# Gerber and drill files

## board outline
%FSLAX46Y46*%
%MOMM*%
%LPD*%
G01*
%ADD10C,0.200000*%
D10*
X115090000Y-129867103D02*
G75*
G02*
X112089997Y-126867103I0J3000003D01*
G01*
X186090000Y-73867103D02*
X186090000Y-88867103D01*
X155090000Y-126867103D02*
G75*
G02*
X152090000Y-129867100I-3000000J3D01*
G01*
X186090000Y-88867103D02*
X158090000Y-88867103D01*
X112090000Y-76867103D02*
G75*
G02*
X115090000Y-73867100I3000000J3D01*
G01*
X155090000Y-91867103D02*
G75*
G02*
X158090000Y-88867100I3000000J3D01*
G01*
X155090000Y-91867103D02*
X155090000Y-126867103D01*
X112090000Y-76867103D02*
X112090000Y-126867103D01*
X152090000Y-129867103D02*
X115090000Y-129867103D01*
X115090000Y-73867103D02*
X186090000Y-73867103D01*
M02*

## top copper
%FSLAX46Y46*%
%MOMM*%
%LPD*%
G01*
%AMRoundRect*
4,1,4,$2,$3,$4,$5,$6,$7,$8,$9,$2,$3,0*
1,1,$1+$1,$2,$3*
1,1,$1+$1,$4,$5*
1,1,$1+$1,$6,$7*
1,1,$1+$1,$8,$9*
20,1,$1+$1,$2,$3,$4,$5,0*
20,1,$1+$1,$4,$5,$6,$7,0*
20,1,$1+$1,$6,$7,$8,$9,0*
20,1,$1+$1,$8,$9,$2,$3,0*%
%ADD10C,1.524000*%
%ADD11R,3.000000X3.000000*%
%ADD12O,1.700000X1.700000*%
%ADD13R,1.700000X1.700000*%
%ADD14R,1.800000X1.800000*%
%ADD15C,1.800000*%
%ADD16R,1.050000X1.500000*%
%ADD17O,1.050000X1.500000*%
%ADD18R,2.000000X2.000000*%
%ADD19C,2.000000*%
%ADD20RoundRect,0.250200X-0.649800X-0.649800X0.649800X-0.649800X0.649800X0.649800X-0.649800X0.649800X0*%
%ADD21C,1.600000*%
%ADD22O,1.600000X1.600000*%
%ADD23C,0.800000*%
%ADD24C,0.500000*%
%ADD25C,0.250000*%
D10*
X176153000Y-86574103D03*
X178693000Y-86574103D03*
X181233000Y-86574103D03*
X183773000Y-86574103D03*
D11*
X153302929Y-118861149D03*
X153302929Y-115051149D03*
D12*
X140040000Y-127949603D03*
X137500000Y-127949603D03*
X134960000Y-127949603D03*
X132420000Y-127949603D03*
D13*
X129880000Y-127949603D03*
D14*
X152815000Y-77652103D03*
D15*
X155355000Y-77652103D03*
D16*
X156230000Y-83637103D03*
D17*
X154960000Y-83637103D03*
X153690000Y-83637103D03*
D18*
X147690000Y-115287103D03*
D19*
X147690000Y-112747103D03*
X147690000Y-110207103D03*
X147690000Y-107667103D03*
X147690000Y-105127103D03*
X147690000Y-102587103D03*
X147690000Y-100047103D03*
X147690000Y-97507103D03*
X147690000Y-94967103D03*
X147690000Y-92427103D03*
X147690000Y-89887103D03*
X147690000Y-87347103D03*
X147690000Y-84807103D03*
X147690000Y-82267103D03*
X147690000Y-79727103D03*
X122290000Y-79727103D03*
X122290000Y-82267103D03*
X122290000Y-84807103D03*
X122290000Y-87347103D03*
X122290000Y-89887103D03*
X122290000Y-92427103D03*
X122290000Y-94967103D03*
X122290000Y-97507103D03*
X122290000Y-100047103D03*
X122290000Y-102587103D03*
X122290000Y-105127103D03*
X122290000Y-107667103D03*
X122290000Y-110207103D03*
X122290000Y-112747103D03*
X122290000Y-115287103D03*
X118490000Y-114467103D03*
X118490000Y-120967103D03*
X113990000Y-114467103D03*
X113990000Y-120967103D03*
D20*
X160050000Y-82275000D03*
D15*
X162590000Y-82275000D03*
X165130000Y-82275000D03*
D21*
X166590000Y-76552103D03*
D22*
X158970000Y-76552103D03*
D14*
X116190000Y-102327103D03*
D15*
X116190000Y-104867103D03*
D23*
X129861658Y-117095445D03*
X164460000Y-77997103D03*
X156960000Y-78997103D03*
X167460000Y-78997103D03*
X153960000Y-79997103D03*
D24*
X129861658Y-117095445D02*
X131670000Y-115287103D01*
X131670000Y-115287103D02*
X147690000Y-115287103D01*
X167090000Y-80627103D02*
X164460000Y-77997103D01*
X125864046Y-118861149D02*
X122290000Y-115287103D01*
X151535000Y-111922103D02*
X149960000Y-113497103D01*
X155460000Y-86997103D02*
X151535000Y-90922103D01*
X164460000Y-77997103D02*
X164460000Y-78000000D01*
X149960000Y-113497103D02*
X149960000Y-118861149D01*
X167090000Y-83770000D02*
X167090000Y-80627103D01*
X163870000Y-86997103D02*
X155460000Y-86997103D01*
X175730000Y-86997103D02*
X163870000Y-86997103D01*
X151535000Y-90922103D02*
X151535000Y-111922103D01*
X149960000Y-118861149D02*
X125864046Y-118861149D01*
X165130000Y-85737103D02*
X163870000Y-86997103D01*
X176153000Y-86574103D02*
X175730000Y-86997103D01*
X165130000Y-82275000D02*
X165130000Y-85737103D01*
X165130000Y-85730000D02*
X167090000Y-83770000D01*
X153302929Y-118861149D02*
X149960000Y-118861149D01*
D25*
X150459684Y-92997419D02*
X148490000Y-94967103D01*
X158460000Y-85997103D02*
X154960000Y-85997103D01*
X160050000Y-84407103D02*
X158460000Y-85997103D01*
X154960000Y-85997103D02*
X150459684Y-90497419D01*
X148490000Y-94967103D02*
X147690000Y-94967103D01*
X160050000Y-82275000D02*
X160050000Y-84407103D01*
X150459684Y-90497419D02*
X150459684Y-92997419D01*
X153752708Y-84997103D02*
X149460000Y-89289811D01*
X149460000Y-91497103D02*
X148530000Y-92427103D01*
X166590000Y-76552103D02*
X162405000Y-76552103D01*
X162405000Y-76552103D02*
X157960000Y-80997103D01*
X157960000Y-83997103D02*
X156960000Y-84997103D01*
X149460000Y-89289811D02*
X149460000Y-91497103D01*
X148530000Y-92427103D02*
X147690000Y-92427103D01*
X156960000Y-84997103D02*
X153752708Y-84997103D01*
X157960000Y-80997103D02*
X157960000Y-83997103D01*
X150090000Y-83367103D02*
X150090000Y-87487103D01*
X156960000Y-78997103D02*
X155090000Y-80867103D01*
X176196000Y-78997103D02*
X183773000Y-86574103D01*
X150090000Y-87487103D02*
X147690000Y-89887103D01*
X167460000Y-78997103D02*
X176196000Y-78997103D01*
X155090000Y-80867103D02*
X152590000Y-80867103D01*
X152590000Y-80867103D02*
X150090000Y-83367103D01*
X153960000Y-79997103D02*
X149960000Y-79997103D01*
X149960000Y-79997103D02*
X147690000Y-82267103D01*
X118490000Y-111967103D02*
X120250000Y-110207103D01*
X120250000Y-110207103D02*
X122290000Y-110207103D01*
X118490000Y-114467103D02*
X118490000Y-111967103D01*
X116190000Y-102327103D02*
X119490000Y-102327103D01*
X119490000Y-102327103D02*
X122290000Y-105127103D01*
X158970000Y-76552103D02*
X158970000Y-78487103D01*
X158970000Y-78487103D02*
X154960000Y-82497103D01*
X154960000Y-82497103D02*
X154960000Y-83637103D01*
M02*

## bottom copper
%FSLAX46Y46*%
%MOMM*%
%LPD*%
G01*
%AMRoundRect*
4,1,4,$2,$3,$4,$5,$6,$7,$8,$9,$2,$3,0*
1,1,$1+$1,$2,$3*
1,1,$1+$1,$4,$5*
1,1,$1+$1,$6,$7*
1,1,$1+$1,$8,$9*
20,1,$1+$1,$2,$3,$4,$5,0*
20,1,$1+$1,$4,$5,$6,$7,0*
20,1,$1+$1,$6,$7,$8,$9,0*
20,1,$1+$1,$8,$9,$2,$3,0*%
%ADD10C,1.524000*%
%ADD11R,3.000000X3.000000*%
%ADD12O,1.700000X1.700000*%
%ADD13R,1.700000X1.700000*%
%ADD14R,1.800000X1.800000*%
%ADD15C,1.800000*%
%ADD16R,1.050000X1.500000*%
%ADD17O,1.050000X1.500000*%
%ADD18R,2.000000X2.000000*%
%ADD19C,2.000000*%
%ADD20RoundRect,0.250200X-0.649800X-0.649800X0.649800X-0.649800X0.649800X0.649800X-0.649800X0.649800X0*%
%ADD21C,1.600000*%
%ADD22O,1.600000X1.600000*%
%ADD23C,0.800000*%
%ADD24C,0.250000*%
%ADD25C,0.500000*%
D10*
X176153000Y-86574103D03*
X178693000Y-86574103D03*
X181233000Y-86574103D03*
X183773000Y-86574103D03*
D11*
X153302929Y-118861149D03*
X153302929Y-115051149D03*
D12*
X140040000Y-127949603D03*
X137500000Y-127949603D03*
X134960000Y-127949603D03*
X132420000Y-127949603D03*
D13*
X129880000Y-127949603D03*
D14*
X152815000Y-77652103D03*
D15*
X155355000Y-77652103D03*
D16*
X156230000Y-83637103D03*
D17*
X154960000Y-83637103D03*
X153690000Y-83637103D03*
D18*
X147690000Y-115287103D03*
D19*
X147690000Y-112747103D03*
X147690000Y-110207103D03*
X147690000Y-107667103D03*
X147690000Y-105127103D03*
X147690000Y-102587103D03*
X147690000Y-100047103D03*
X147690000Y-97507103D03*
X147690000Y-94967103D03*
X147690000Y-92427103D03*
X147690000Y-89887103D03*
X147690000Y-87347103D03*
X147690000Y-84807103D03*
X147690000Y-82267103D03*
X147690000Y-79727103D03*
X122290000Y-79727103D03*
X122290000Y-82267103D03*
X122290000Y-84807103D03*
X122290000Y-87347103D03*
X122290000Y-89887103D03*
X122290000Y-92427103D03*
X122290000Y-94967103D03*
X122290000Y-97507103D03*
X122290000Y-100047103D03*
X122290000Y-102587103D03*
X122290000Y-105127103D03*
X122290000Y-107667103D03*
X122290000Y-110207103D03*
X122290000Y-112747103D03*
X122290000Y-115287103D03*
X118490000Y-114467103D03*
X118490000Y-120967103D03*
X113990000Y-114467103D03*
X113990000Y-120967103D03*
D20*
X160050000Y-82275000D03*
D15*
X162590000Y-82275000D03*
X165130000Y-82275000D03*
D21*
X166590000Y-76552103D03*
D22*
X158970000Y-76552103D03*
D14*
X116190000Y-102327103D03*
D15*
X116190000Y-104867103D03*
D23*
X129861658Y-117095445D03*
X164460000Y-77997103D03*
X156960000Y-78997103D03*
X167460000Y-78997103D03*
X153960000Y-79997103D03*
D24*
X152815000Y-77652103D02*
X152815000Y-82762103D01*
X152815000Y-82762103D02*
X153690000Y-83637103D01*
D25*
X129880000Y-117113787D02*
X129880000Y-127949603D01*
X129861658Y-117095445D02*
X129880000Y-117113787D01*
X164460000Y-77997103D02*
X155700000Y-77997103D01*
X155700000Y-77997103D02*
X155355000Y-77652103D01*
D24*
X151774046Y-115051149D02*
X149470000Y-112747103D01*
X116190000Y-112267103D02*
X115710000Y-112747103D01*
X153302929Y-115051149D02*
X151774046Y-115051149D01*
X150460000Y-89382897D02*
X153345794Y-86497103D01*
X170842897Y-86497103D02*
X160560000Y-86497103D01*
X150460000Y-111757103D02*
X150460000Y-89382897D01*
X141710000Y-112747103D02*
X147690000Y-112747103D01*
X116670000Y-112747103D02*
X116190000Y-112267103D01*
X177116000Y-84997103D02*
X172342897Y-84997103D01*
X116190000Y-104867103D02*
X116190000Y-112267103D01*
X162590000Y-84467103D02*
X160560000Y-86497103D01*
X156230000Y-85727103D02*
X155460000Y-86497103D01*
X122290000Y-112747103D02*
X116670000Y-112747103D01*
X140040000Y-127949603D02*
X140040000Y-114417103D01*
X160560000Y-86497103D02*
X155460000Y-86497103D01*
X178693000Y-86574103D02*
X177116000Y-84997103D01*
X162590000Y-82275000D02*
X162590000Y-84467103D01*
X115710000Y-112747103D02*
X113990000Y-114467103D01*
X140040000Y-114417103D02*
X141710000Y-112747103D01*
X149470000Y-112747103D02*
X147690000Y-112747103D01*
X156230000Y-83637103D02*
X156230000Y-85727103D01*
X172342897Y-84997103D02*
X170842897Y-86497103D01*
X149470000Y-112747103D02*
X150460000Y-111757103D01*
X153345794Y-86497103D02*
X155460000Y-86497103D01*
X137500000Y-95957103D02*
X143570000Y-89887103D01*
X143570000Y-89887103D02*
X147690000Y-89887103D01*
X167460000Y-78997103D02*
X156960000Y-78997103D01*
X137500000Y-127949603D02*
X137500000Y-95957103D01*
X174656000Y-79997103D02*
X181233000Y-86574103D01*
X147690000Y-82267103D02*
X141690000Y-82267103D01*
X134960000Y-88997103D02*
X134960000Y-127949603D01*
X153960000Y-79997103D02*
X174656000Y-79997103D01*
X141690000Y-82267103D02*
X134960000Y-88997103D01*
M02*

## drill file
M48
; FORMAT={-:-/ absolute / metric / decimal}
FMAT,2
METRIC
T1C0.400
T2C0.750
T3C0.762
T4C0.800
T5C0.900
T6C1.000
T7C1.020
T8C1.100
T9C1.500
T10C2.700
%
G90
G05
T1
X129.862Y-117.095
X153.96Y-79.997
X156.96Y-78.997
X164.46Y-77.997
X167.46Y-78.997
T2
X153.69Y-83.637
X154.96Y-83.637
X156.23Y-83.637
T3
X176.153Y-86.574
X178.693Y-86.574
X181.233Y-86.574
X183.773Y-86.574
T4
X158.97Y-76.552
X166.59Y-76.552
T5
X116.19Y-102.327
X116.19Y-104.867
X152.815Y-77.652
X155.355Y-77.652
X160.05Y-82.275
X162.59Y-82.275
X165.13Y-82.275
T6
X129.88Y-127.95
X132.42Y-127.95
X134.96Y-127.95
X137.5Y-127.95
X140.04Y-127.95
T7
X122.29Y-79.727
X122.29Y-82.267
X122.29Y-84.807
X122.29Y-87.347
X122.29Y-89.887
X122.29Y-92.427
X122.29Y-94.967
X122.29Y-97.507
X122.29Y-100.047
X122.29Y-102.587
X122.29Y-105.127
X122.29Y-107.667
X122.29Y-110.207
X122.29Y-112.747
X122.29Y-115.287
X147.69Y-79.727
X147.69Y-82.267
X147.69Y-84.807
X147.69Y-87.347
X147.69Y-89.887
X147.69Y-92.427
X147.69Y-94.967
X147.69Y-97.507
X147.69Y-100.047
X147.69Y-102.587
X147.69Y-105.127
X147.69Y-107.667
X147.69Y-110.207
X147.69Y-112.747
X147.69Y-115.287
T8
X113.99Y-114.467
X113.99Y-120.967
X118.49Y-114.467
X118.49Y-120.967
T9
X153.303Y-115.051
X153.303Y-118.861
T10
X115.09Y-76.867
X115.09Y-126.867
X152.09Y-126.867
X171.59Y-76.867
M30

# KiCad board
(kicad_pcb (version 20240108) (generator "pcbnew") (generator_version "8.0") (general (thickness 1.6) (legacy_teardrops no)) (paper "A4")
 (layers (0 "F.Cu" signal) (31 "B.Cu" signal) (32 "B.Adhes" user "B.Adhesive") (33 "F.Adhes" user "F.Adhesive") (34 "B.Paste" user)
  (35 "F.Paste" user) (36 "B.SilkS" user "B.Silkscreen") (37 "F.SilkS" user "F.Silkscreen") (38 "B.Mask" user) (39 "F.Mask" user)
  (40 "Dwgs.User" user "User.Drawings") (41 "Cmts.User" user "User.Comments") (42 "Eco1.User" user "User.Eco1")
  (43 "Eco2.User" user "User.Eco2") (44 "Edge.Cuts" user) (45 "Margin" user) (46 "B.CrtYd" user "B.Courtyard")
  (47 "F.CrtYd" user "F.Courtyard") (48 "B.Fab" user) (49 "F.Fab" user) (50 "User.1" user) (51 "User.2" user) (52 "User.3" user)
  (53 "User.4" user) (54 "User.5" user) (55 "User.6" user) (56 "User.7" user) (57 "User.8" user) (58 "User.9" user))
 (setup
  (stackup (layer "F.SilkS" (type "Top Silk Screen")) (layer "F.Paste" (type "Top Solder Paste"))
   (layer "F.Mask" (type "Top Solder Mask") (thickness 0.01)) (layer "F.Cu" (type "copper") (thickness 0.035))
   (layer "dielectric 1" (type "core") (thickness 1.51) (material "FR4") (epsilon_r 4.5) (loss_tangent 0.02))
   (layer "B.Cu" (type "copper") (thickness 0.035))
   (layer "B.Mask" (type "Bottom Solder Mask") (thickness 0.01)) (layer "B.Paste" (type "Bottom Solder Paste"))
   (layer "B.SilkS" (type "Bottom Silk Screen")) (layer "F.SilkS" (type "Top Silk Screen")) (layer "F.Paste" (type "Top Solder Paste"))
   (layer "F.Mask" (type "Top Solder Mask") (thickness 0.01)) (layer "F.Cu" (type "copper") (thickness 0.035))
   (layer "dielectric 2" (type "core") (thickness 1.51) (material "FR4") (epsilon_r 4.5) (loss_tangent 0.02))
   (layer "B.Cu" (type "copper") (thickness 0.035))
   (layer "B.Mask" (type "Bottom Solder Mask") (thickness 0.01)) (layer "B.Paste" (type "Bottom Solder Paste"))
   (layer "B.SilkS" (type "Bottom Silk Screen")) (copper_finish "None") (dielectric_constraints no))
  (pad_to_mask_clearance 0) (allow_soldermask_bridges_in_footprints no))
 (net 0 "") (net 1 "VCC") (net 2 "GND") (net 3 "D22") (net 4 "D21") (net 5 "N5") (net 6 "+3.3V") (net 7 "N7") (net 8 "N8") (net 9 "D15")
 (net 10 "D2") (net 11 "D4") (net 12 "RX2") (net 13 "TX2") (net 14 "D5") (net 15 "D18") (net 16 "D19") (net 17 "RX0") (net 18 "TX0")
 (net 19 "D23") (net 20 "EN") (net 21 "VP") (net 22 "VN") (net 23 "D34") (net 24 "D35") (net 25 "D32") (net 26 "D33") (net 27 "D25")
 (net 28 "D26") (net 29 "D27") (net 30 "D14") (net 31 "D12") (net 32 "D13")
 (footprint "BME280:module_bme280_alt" (layer "F.Cu") (at 183.773 86.574103 90)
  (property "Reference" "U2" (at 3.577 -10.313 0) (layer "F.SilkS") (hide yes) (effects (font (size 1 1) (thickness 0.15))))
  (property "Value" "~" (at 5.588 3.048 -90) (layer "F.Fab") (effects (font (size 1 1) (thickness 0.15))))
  (pad "1" thru_hole circle (at 0 -7.62 90) (size 1.524 1.524) (drill 0.762) (layers "*.Cu" "*.Mask") (remove_unused_layers no)
   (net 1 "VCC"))
  (pad "2" thru_hole circle (at 0 -5.08 90) (size 1.524 1.524) (drill 0.762) (layers "*.Cu" "*.Mask") (remove_unused_layers no)
   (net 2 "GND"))
  (pad "3" thru_hole circle (at 0 -2.54 90) (size 1.524 1.524) (drill 0.762) (layers "*.Cu" "*.Mask") (remove_unused_layers no)
   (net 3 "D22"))
  (pad "4" thru_hole circle (at 0 0 90) (size 1.524 1.524) (drill 0.762) (layers "*.Cu" "*.Mask") (remove_unused_layers no) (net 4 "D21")))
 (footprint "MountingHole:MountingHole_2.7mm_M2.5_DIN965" (layer "F.Cu") (at 115.09 76.867103)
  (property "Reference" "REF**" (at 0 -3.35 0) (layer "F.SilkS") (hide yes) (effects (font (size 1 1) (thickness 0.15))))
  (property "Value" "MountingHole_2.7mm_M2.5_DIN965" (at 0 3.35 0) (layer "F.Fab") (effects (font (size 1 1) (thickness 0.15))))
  (pad "" np_thru_hole circle (at 0 0) (size 2.7 2.7) (drill 2.7) (layers "F&B.Cu" "*.Mask")))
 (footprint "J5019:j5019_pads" (layer "F.Cu") (at 149.492929 116.321149 90)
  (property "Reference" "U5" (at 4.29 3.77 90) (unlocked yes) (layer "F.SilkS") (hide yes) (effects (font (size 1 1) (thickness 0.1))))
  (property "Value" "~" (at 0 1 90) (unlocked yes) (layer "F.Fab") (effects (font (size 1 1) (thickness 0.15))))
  (pad "3" thru_hole rect (at -2.54 3.81 180) (size 3 3) (drill 1.5) (layers "*.Cu" "*.Mask") (remove_unused_layers no) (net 1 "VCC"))
  (pad "4" thru_hole rect (at 1.27 3.81 180) (size 3 3) (drill 1.5) (layers "*.Cu" "*.Mask") (remove_unused_layers no) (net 2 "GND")))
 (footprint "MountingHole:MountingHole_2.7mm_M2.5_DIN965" (layer "F.Cu") (at 171.59 76.867103)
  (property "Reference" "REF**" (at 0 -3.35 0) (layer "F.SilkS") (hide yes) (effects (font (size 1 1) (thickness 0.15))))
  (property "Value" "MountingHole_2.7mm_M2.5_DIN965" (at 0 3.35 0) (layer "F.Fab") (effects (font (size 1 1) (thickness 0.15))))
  (pad "" np_thru_hole circle (at 0 0) (size 2.7 2.7) (drill 2.7) (layers "F&B.Cu" "*.Mask")))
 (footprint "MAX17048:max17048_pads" (layer "F.Cu") (at 136.23 131.759603 180)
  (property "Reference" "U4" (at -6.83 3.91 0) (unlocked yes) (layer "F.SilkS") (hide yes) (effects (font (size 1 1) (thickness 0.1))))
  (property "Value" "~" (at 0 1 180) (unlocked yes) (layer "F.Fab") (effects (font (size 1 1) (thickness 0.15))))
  (pad "1" thru_hole oval (at -3.81 3.81 270) (size 1.7 1.7) (drill 1) (layers "*.Cu" "*.Mask") (remove_unused_layers no) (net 2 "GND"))
  (pad "2" thru_hole oval (at -1.27 3.81 270) (size 1.7 1.7) (drill 1) (layers "*.Cu" "*.Mask") (remove_unused_layers no) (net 4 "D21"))
  (pad "3" thru_hole oval (at 1.27 3.81 270) (size 1.7 1.7) (drill 1) (layers "*.Cu" "*.Mask") (remove_unused_layers no) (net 3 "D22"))
  (pad "4" thru_hole oval (at 3.81 3.81 270) (size 1.7 1.7) (drill 1) (layers "*.Cu" "*.Mask") (remove_unused_layers no) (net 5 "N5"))
  (pad "5" thru_hole rect (at 6.35 3.81 270) (size 1.7 1.7) (drill 1) (layers "*.Cu" "*.Mask") (remove_unused_layers no) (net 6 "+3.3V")))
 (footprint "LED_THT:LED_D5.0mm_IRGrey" (layer "F.Cu") (at 152.815 77.652103)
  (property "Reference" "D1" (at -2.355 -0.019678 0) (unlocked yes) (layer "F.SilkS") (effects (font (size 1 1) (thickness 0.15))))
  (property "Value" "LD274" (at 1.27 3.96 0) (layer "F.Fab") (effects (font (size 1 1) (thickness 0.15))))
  (pad "1" thru_hole rect (at 0 0) (size 1.8 1.8) (drill 0.9) (layers "*.Cu" "*.Mask") (remove_unused_layers no) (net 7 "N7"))
  (pad "2" thru_hole circle (at 2.54 0) (size 1.8 1.8) (drill 0.9) (layers "*.Cu" "*.Mask") (remove_unused_layers no) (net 1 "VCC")))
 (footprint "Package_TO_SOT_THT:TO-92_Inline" (layer "F.Cu") (at 156.23 83.637103 180)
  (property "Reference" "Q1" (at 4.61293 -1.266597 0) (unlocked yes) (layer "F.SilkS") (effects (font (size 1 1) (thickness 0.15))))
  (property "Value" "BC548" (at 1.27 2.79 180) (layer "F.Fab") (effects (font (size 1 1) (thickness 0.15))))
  (pad "1" thru_hole rect (at 0 0 180) (size 1.05 1.5) (drill 0.75) (layers "*.Cu" "*.Mask") (remove_unused_layers no) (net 2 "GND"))
  (pad "2" thru_hole oval (at 1.27 0 180) (size 1.05 1.5) (drill 0.75) (layers "*.Cu" "*.Mask") (remove_unused_layers no) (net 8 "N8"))
  (pad "3" thru_hole oval (at 2.54 0 180) (size 1.05 1.5) (drill 0.75) (layers "*.Cu" "*.Mask") (remove_unused_layers no) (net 7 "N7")))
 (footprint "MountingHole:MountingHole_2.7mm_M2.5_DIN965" (layer "F.Cu") (at 115.09 126.867103)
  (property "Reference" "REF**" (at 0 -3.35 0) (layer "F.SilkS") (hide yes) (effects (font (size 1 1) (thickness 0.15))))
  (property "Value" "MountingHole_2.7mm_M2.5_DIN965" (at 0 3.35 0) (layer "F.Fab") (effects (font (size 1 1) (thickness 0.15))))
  (pad "" np_thru_hole circle (at 0 0) (size 2.7 2.7) (drill 2.7) (layers "F&B.Cu" "*.Mask")))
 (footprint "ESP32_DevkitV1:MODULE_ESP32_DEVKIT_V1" (layer "F.Cu") (at 134.99 99.772103 180)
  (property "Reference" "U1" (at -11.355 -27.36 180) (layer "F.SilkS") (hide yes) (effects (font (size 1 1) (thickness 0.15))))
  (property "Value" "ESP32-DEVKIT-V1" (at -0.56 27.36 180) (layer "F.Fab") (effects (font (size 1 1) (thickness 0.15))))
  (pad "1" thru_hole rect (at -12.7 -15.515 180) (size 2 2) (drill 1.02) (layers "*.Cu" "*.Mask") (remove_unused_layers no) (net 6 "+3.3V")
   (solder_mask_margin 0.102))
  (pad "2" thru_hole circle (at -12.7 -12.975 180) (size 2 2) (drill 1.02) (layers "*.Cu" "*.Mask") (remove_unused_layers no) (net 2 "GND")
   (solder_mask_margin 0.102))
  (pad "3" thru_hole circle (at -12.7 -10.435 180) (size 2 2) (drill 1.02) (layers "*.Cu" "*.Mask") (remove_unused_layers no) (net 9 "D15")
   (solder_mask_margin 0.102))
  (pad "4" thru_hole circle (at -12.7 -7.895 180) (size 2 2) (drill 1.02) (layers "*.Cu" "*.Mask") (remove_unused_layers no) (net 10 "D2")
   (solder_mask_margin 0.102))
  (pad "5" thru_hole circle (at -12.7 -5.355 180) (size 2 2) (drill 1.02) (layers "*.Cu" "*.Mask") (remove_unused_layers no) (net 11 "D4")
   (solder_mask_margin 0.102))
  (pad "6" thru_hole circle (at -12.7 -2.815 180) (size 2 2) (drill 1.02) (layers "*.Cu" "*.Mask") (remove_unused_layers no) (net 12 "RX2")
   (solder_mask_margin 0.102))
  (pad "7" thru_hole circle (at -12.7 -0.275 180) (size 2 2) (drill 1.02) (layers "*.Cu" "*.Mask") (remove_unused_layers no) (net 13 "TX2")
   (solder_mask_margin 0.102))
  (pad "8" thru_hole circle (at -12.7 2.265 180) (size 2 2) (drill 1.02) (layers "*.Cu" "*.Mask") (remove_unused_layers no) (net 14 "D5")
   (solder_mask_margin 0.102))
  (pad "9" thru_hole circle (at -12.7 4.805 180) (size 2 2) (drill 1.02) (layers "*.Cu" "*.Mask") (remove_unused_layers no) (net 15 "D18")
   (solder_mask_margin 0.102))
  (pad "10" thru_hole circle (at -12.7 7.345 180) (size 2 2) (drill 1.02) (layers "*.Cu" "*.Mask") (remove_unused_layers no) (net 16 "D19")
   (solder_mask_margin 0.102))
  (pad "11" thru_hole circle (at -12.7 9.885 180) (size 2 2) (drill 1.02) (layers "*.Cu" "*.Mask") (remove_unused_layers no) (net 4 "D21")
   (solder_mask_margin 0.102))
  (pad "12" thru_hole circle (at -12.7 12.425 180) (size 2 2) (drill 1.02) (layers "*.Cu" "*.Mask") (remove_unused_layers no) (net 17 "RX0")
   (solder_mask_margin 0.102))
  (pad "13" thru_hole circle (at -12.7 14.965 180) (size 2 2) (drill 1.02) (layers "*.Cu" "*.Mask") (remove_unused_layers no) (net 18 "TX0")
   (solder_mask_margin 0.102))
  (pad "14" thru_hole circle (at -12.7 17.505 180) (size 2 2) (drill 1.02) (layers "*.Cu" "*.Mask") (remove_unused_layers no) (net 3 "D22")
   (solder_mask_margin 0.102))
  (pad "15" thru_hole circle (at -12.7 20.045 180) (size 2 2) (drill 1.02) (layers "*.Cu" "*.Mask") (remove_unused_layers no) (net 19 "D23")
   (solder_mask_margin 0.102))
  (pad "16" thru_hole circle (at 12.7 20.045 180) (size 2 2) (drill 1.02) (layers "*.Cu" "*.Mask") (remove_unused_layers no) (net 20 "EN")
   (solder_mask_margin 0.102))
  (pad "17" thru_hole circle (at 12.7 17.505 180) (size 2 2) (drill 1.02) (layers "*.Cu" "*.Mask") (remove_unused_layers no) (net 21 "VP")
   (solder_mask_margin 0.102))
  (pad "18" thru_hole circle (at 12.7 14.965 180) (size 2 2) (drill 1.02) (layers "*.Cu" "*.Mask") (remove_unused_layers no) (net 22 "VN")
   (solder_mask_margin 0.102))
  (pad "19" thru_hole circle (at 12.7 12.425 180) (size 2 2) (drill 1.02) (layers "*.Cu" "*.Mask") (remove_unused_layers no) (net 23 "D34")
   (solder_mask_margin 0.102))
  (pad "20" thru_hole circle (at 12.7 9.885 180) (size 2 2) (drill 1.02) (layers "*.Cu" "*.Mask") (remove_unused_layers no) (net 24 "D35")
   (solder_mask_margin 0.102))
  (pad "21" thru_hole circle (at 12.7 7.345 180) (size 2 2) (drill 1.02) (layers "*.Cu" "*.Mask") (remove_unused_layers no) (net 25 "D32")
   (solder_mask_margin 0.102))
  (pad "22" thru_hole circle (at 12.7 4.805 180) (size 2 2) (drill 1.02) (layers "*.Cu" "*.Mask") (remove_unused_layers no) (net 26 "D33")
   (solder_mask_margin 0.102))
  (pad "23" thru_hole circle (at 12.7 2.265 180) (size 2 2) (drill 1.02) (layers "*.Cu" "*.Mask") (remove_unused_layers no) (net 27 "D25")
   (solder_mask_margin 0.102))
  (pad "24" thru_hole circle (at 12.7 -0.275 180) (size 2 2) (drill 1.02) (layers "*.Cu" "*.Mask") (remove_unused_layers no) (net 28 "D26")
   (solder_mask_margin 0.102))
  (pad "25" thru_hole circle (at 12.7 -2.815 180) (size 2 2) (drill 1.02) (layers "*.Cu" "*.Mask") (remove_unused_layers no) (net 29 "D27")
   (solder_mask_margin 0.102))
  (pad "26" thru_hole circle (at 12.7 -5.355 180) (size 2 2) (drill 1.02) (layers "*.Cu" "*.Mask") (remove_unused_layers no) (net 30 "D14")
   (solder_mask_margin 0.102))
  (pad "27" thru_hole circle (at 12.7 -7.895 180) (size 2 2) (drill 1.02) (layers "*.Cu" "*.Mask") (remove_unused_layers no) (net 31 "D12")
   (solder_mask_margin 0.102))
  (pad "28" thru_hole circle (at 12.7 -10.435 180) (size 2 2) (drill 1.02) (layers "*.Cu" "*.Mask") (remove_unused_layers no) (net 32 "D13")
   (solder_mask_margin 0.102))
  (pad "29" thru_hole circle (at 12.7 -12.975 180) (size 2 2) (drill 1.02) (layers "*.Cu" "*.Mask") (remove_unused_layers no) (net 2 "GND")
   (solder_mask_margin 0.102))
  (pad "30" thru_hole circle (at 12.7 -15.515 180) (size 2 2) (drill 1.02) (layers "*.Cu" "*.Mask") (remove_unused_layers no) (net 1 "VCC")
   (solder_mask_margin 0.102))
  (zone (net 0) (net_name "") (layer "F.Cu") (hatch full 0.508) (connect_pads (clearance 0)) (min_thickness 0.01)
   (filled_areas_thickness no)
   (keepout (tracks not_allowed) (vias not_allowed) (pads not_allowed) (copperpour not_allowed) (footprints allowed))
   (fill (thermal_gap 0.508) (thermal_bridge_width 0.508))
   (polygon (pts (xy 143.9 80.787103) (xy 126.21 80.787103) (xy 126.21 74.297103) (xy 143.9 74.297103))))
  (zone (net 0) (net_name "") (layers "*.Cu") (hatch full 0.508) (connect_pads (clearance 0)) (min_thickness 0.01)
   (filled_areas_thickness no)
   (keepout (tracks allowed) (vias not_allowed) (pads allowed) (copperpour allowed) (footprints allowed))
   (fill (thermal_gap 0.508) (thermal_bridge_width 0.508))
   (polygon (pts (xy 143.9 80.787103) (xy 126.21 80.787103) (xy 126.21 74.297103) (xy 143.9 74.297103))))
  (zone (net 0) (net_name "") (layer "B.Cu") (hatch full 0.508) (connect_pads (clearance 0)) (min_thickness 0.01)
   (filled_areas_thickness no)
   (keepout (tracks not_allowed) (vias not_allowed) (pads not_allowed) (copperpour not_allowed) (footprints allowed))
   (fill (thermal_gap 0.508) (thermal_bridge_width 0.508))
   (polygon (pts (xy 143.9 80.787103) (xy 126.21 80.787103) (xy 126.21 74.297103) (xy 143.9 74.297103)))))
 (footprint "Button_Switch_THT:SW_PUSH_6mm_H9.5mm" (layer "F.Cu") (at 118.49 114.467103 -90)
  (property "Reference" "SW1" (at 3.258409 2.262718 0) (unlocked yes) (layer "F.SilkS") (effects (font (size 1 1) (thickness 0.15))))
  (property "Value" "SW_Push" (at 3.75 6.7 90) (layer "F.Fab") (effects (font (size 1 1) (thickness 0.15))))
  (pad "1" thru_hole circle (at 0 0) (size 2 2) (drill 1.1) (layers "*.Cu" "*.Mask") (remove_unused_layers no) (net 32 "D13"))
  (pad "1" thru_hole circle (at 6.5 0) (size 2 2) (drill 1.1) (layers "*.Cu" "*.Mask") (remove_unused_layers no) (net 32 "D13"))
  (pad "2" thru_hole circle (at 0 4.5) (size 2 2) (drill 1.1) (layers "*.Cu" "*.Mask") (remove_unused_layers no) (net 2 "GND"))
  (pad "2" thru_hole circle (at 6.5 4.5) (size 2 2) (drill 1.1) (layers "*.Cu" "*.Mask") (remove_unused_layers no) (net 2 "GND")))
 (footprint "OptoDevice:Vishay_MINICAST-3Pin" (layer "F.Cu") (at 160.05 82.275)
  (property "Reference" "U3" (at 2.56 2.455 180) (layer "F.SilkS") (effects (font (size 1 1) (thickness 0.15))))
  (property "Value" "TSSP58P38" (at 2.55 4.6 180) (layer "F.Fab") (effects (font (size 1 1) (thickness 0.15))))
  (pad "1" thru_hole roundrect (at 0 0) (size 1.8 1.8) (drill 0.9) (layers "*.Cu" "*.Mask") (remove_unused_layers no)
   (roundrect_rratio 0.139) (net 15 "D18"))
  (pad "2" thru_hole circle (at 2.54 0) (size 1.8 1.8) (drill 0.9) (layers "*.Cu" "*.Mask") (remove_unused_layers no) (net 2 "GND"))
  (pad "3" thru_hole circle (at 5.08 0) (size 1.8 1.8) (drill 0.9) (layers "*.Cu" "*.Mask") (remove_unused_layers no) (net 1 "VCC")))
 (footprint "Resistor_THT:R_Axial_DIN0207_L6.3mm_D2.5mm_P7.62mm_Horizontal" (layer "F.Cu") (at 166.59 76.552103 180)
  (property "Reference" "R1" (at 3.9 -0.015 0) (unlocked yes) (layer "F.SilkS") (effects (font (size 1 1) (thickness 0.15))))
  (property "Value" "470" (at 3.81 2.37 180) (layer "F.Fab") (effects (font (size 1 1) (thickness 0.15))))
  (pad "1" thru_hole circle (at 0 0 180) (size 1.6 1.6) (drill 0.8) (layers "*.Cu" "*.Mask") (remove_unused_layers no) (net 16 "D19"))
  (pad "2" thru_hole oval (at 7.62 0 180) (size 1.6 1.6) (drill 0.8) (layers "*.Cu" "*.Mask") (remove_unused_layers no) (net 8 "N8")))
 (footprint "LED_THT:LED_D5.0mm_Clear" (layer "F.Cu") (at 116.19 102.327103 -90)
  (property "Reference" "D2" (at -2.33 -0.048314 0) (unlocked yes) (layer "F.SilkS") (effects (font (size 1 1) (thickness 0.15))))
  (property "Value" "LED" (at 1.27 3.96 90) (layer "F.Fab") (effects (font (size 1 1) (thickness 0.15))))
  (pad "1" thru_hole rect (at 0 0 270) (size 1.8 1.8) (drill 0.9) (layers "*.Cu" "*.Mask") (remove_unused_layers no) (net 30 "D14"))
  (pad "2" thru_hole circle (at 2.54 0 270) (size 1.8 1.8) (drill 0.9) (layers "*.Cu" "*.Mask") (remove_unused_layers no) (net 2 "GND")))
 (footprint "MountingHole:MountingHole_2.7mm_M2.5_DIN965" (layer "F.Cu") (at 152.09 126.867103)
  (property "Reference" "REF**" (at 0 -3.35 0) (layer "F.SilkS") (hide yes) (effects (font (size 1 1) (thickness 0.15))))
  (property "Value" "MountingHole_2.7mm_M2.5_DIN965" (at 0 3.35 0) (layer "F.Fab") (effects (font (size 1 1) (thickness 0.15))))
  (pad "" np_thru_hole circle (at 0 0) (size 2.7 2.7) (drill 2.7) (layers "*.Cu" "*.Mask")))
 (gr_arc (start 115.09 129.867103) (mid 112.96868 128.988423) (end 112.09 126.867103) (stroke (width 0.2) (type default))
  (layer "Edge.Cuts"))
 (gr_line (start 186.09 73.867103) (end 186.09 88.867103) (stroke (width 0.2) (type default)) (layer "Edge.Cuts"))
 (gr_arc (start 155.09 126.867103) (mid 154.21132 128.988423) (end 152.09 129.867103) (stroke (width 0.2) (type default))
  (layer "Edge.Cuts"))
 (gr_line (start 186.09 88.867103) (end 158.09 88.867103) (stroke (width 0.2) (type default)) (layer "Edge.Cuts"))
 (gr_arc (start 112.09 76.867103) (mid 112.96868 74.745783) (end 115.09 73.867103) (stroke (width 0.2) (type default)) (layer "Edge.Cuts"))
 (gr_arc (start 155.09 91.867103) (mid 155.96868 89.745783) (end 158.09 88.867103) (stroke (width 0.2) (type default)) (layer "Edge.Cuts"))
 (gr_line (start 155.09 91.867103) (end 155.09 126.867103) (stroke (width 0.2) (type default)) (layer "Edge.Cuts"))
 (gr_line (start 112.09 76.867103) (end 112.09 126.867103) (stroke (width 0.2) (type default)) (layer "Edge.Cuts"))
 (gr_line (start 152.09 129.867103) (end 115.09 129.867103) (stroke (width 0.2) (type default)) (layer "Edge.Cuts"))
 (gr_line (start 115.09 73.867103) (end 186.09 73.867103) (stroke (width 0.2) (type default)) (layer "Edge.Cuts"))
 (segment (start 152.815 77.652103) (end 152.815 82.762103) (width 0.25) (layer "B.Cu") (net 7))
 (segment (start 152.815 82.762103) (end 153.69 83.637103) (width 0.25) (layer "B.Cu") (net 7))
 (segment (start 129.861658 117.095445) (end 131.67 115.287103) (width 0.5) (layer "F.Cu") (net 6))
 (segment (start 131.67 115.287103) (end 147.69 115.287103) (width 0.5) (layer "F.Cu") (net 6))
 (via (at 129.861658 117.095445) (size 0.8) (drill 0.4) (layers "F.Cu" "B.Cu") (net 6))
 (segment (start 129.88 117.113787) (end 129.88 127.949603) (width 0.5) (layer "B.Cu") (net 6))
 (segment (start 129.861658 117.095445) (end 129.88 117.113787) (width 0.5) (layer "B.Cu") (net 6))
 (segment (start 167.09 80.627103) (end 164.46 77.997103) (width 0.5) (layer "F.Cu") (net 1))
 (segment (start 125.864046 118.861149) (end 122.29 115.287103) (width 0.5) (layer "F.Cu") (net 1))
 (segment (start 151.535 111.922103) (end 149.96 113.497103) (width 0.5) (layer "F.Cu") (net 1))
 (segment (start 155.46 86.997103) (end 151.535 90.922103) (width 0.5) (layer "F.Cu") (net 1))
 (segment (start 164.46 77.997103) (end 164.46 78) (width 0.5) (layer "F.Cu") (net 1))
 (segment (start 149.96 113.497103) (end 149.96 118.861149) (width 0.5) (layer "F.Cu") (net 1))
 (segment (start 167.09 83.77) (end 167.09 80.627103) (width 0.5) (layer "F.Cu") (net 1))
 (segment (start 163.87 86.997103) (end 155.46 86.997103) (width 0.5) (layer "F.Cu") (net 1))
 (segment (start 175.73 86.997103) (end 163.87 86.997103) (width 0.5) (layer "F.Cu") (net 1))
 (segment (start 151.535 90.922103) (end 151.535 111.922103) (width 0.5) (layer "F.Cu") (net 1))
 (segment (start 149.96 118.861149) (end 125.864046 118.861149) (width 0.5) (layer "F.Cu") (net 1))
 (segment (start 165.13 85.737103) (end 163.87 86.997103) (width 0.5) (layer "F.Cu") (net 1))
 (segment (start 176.153 86.574103) (end 175.73 86.997103) (width 0.5) (layer "F.Cu") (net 1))
 (segment (start 165.13 82.275) (end 165.13 85.737103) (width 0.5) (layer "F.Cu") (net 1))
 (segment (start 165.13 85.73) (end 167.09 83.77) (width 0.5) (layer "F.Cu") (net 1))
 (segment (start 153.302929 118.861149) (end 149.96 118.861149) (width 0.5) (layer "F.Cu") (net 1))
 (via (at 164.46 77.997103) (size 0.8) (drill 0.4) (layers "F.Cu" "B.Cu") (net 1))
 (segment (start 164.46 77.997103) (end 155.7 77.997103) (width 0.5) (layer "B.Cu") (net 1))
 (segment (start 155.7 77.997103) (end 155.355 77.652103) (width 0.5) (layer "B.Cu") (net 1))
 (segment (start 151.774046 115.051149) (end 149.47 112.747103) (width 0.25) (layer "B.Cu") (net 2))
 (segment (start 116.19 112.267103) (end 115.71 112.747103) (width 0.25) (layer "B.Cu") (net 2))
 (segment (start 153.302929 115.051149) (end 151.774046 115.051149) (width 0.25) (layer "B.Cu") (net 2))
 (segment (start 150.46 89.382897) (end 153.345794 86.497103) (width 0.25) (layer "B.Cu") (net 2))
 (segment (start 170.842897 86.497103) (end 160.56 86.497103) (width 0.25) (layer "B.Cu") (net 2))
 (segment (start 150.46 111.757103) (end 150.46 89.382897) (width 0.25) (layer "B.Cu") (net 2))
 (segment (start 141.71 112.747103) (end 147.69 112.747103) (width 0.25) (layer "B.Cu") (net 2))
 (segment (start 116.67 112.747103) (end 116.19 112.267103) (width 0.25) (layer "B.Cu") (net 2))
 (segment (start 177.116 84.997103) (end 172.342897 84.997103) (width 0.25) (layer "B.Cu") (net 2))
 (segment (start 116.19 104.867103) (end 116.19 112.267103) (width 0.25) (layer "B.Cu") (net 2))
 (segment (start 162.59 84.467103) (end 160.56 86.497103) (width 0.25) (layer "B.Cu") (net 2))
 (segment (start 156.23 85.727103) (end 155.46 86.497103) (width 0.25) (layer "B.Cu") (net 2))
 (segment (start 122.29 112.747103) (end 116.67 112.747103) (width 0.25) (layer "B.Cu") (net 2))
 (segment (start 140.04 127.949603) (end 140.04 114.417103) (width 0.25) (layer "B.Cu") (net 2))
 (segment (start 160.56 86.497103) (end 155.46 86.497103) (width 0.25) (layer "B.Cu") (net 2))
 (segment (start 178.693 86.574103) (end 177.116 84.997103) (width 0.25) (layer "B.Cu") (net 2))
 (segment (start 162.59 82.275) (end 162.59 84.467103) (width 0.25) (layer "B.Cu") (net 2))
 (segment (start 115.71 112.747103) (end 113.99 114.467103) (width 0.25) (layer "B.Cu") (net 2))
 (segment (start 140.04 114.417103) (end 141.71 112.747103) (width 0.25) (layer "B.Cu") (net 2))
 (segment (start 149.47 112.747103) (end 147.69 112.747103) (width 0.25) (layer "B.Cu") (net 2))
 (segment (start 156.23 83.637103) (end 156.23 85.727103) (width 0.25) (layer "B.Cu") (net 2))
 (segment (start 172.342897 84.997103) (end 170.842897 86.497103) (width 0.25) (layer "B.Cu") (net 2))
 (segment (start 149.47 112.747103) (end 150.46 111.757103) (width 0.25) (layer "B.Cu") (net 2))
 (segment (start 153.345794 86.497103) (end 155.46 86.497103) (width 0.25) (layer "B.Cu") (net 2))
 (segment (start 150.459684 92.997419) (end 148.49 94.967103) (width 0.25) (layer "F.Cu") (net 15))
 (segment (start 158.46 85.997103) (end 154.96 85.997103) (width 0.25) (layer "F.Cu") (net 15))
 (segment (start 160.05 84.407103) (end 158.46 85.997103) (width 0.25) (layer "F.Cu") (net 15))
 (segment (start 154.96 85.997103) (end 150.459684 90.497419) (width 0.25) (layer "F.Cu") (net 15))
 (segment (start 148.49 94.967103) (end 147.69 94.967103) (width 0.25) (layer "F.Cu") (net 15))
 (segment (start 160.05 82.275) (end 160.05 84.407103) (width 0.25) (layer "F.Cu") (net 15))
 (segment (start 150.459684 90.497419) (end 150.459684 92.997419) (width 0.25) (layer "F.Cu") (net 15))
 (segment (start 153.752708 84.997103) (end 149.46 89.289811) (width 0.25) (layer "F.Cu") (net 16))
 (segment (start 149.46 91.497103) (end 148.53 92.427103) (width 0.25) (layer "F.Cu") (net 16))
 (segment (start 166.59 76.552103) (end 162.405 76.552103) (width 0.25) (layer "F.Cu") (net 16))
 (segment (start 162.405 76.552103) (end 157.96 80.997103) (width 0.25) (layer "F.Cu") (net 16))
 (segment (start 157.96 83.997103) (end 156.96 84.997103) (width 0.25) (layer "F.Cu") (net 16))
 (segment (start 149.46 89.289811) (end 149.46 91.497103) (width 0.25) (layer "F.Cu") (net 16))
 (segment (start 148.53 92.427103) (end 147.69 92.427103) (width 0.25) (layer "F.Cu") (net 16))
 (segment (start 156.96 84.997103) (end 153.752708 84.997103) (width 0.25) (layer "F.Cu") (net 16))
 (segment (start 157.96 80.997103) (end 157.96 83.997103) (width 0.25) (layer "F.Cu") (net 16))
 (segment (start 150.09 83.367103) (end 150.09 87.487103) (width 0.25) (layer "F.Cu") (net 4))
 (segment (start 156.96 78.997103) (end 155.09 80.867103) (width 0.25) (layer "F.Cu") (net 4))
 (segment (start 176.196 78.997103) (end 183.773 86.574103) (width 0.25) (layer "F.Cu") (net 4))
 (segment (start 150.09 87.487103) (end 147.69 89.887103) (width 0.25) (layer "F.Cu") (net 4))
 (segment (start 167.46 78.997103) (end 176.196 78.997103) (width 0.25) (layer "F.Cu") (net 4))
 (segment (start 155.09 80.867103) (end 152.59 80.867103) (width 0.25) (layer "F.Cu") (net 4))
 (segment (start 152.59 80.867103) (end 150.09 83.367103) (width 0.25) (layer "F.Cu") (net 4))
 (via (at 156.96 78.997103) (size 0.8) (drill 0.4) (layers "F.Cu" "B.Cu") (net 4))
 (via (at 167.46 78.997103) (size 0.8) (drill 0.4) (layers "F.Cu" "B.Cu") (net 4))
 (segment (start 137.5 95.957103) (end 143.57 89.887103) (width 0.25) (layer "B.Cu") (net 4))
 (segment (start 143.57 89.887103) (end 147.69 89.887103) (width 0.25) (layer "B.Cu") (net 4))
 (segment (start 167.46 78.997103) (end 156.96 78.997103) (width 0.25) (layer "B.Cu") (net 4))
 (segment (start 137.5 127.949603) (end 137.5 95.957103) (width 0.25) (layer "B.Cu") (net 4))
 (segment (start 153.96 79.997103) (end 149.96 79.997103) (width 0.25) (layer "F.Cu") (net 3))
 (segment (start 149.96 79.997103) (end 147.69 82.267103) (width 0.25) (layer "F.Cu") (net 3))
 (via (at 153.96 79.997103) (size 0.8) (drill 0.4) (layers "F.Cu" "B.Cu") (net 3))
 (segment (start 174.656 79.997103) (end 181.233 86.574103) (width 0.25) (layer "B.Cu") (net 3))
 (segment (start 147.69 82.267103) (end 141.69 82.267103) (width 0.25) (layer "B.Cu") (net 3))
 (segment (start 134.96 88.997103) (end 134.96 127.949603) (width 0.25) (layer "B.Cu") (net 3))
 (segment (start 153.96 79.997103) (end 174.656 79.997103) (width 0.25) (layer "B.Cu") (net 3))
 (segment (start 141.69 82.267103) (end 134.96 88.997103) (width 0.25) (layer "B.Cu") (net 3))
 (segment (start 118.49 111.967103) (end 120.25 110.207103) (width 0.25) (layer "F.Cu") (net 32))
 (segment (start 120.25 110.207103) (end 122.29 110.207103) (width 0.25) (layer "F.Cu") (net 32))
 (segment (start 118.49 114.467103) (end 118.49 111.967103) (width 0.25) (layer "F.Cu") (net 32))
 (segment (start 116.19 102.327103) (end 119.49 102.327103) (width 0.25) (layer "F.Cu") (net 30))
 (segment (start 119.49 102.327103) (end 122.29 105.127103) (width 0.25) (layer "F.Cu") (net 30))
 (segment (start 158.97 76.552103) (end 158.97 78.487103) (width 0.25) (layer "F.Cu") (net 8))
 (segment (start 158.97 78.487103) (end 154.96 82.497103) (width 0.25) (layer "F.Cu") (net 8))
 (segment (start 154.96 82.497103) (end 154.96 83.637103) (width 0.25) (layer "F.Cu") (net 8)))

